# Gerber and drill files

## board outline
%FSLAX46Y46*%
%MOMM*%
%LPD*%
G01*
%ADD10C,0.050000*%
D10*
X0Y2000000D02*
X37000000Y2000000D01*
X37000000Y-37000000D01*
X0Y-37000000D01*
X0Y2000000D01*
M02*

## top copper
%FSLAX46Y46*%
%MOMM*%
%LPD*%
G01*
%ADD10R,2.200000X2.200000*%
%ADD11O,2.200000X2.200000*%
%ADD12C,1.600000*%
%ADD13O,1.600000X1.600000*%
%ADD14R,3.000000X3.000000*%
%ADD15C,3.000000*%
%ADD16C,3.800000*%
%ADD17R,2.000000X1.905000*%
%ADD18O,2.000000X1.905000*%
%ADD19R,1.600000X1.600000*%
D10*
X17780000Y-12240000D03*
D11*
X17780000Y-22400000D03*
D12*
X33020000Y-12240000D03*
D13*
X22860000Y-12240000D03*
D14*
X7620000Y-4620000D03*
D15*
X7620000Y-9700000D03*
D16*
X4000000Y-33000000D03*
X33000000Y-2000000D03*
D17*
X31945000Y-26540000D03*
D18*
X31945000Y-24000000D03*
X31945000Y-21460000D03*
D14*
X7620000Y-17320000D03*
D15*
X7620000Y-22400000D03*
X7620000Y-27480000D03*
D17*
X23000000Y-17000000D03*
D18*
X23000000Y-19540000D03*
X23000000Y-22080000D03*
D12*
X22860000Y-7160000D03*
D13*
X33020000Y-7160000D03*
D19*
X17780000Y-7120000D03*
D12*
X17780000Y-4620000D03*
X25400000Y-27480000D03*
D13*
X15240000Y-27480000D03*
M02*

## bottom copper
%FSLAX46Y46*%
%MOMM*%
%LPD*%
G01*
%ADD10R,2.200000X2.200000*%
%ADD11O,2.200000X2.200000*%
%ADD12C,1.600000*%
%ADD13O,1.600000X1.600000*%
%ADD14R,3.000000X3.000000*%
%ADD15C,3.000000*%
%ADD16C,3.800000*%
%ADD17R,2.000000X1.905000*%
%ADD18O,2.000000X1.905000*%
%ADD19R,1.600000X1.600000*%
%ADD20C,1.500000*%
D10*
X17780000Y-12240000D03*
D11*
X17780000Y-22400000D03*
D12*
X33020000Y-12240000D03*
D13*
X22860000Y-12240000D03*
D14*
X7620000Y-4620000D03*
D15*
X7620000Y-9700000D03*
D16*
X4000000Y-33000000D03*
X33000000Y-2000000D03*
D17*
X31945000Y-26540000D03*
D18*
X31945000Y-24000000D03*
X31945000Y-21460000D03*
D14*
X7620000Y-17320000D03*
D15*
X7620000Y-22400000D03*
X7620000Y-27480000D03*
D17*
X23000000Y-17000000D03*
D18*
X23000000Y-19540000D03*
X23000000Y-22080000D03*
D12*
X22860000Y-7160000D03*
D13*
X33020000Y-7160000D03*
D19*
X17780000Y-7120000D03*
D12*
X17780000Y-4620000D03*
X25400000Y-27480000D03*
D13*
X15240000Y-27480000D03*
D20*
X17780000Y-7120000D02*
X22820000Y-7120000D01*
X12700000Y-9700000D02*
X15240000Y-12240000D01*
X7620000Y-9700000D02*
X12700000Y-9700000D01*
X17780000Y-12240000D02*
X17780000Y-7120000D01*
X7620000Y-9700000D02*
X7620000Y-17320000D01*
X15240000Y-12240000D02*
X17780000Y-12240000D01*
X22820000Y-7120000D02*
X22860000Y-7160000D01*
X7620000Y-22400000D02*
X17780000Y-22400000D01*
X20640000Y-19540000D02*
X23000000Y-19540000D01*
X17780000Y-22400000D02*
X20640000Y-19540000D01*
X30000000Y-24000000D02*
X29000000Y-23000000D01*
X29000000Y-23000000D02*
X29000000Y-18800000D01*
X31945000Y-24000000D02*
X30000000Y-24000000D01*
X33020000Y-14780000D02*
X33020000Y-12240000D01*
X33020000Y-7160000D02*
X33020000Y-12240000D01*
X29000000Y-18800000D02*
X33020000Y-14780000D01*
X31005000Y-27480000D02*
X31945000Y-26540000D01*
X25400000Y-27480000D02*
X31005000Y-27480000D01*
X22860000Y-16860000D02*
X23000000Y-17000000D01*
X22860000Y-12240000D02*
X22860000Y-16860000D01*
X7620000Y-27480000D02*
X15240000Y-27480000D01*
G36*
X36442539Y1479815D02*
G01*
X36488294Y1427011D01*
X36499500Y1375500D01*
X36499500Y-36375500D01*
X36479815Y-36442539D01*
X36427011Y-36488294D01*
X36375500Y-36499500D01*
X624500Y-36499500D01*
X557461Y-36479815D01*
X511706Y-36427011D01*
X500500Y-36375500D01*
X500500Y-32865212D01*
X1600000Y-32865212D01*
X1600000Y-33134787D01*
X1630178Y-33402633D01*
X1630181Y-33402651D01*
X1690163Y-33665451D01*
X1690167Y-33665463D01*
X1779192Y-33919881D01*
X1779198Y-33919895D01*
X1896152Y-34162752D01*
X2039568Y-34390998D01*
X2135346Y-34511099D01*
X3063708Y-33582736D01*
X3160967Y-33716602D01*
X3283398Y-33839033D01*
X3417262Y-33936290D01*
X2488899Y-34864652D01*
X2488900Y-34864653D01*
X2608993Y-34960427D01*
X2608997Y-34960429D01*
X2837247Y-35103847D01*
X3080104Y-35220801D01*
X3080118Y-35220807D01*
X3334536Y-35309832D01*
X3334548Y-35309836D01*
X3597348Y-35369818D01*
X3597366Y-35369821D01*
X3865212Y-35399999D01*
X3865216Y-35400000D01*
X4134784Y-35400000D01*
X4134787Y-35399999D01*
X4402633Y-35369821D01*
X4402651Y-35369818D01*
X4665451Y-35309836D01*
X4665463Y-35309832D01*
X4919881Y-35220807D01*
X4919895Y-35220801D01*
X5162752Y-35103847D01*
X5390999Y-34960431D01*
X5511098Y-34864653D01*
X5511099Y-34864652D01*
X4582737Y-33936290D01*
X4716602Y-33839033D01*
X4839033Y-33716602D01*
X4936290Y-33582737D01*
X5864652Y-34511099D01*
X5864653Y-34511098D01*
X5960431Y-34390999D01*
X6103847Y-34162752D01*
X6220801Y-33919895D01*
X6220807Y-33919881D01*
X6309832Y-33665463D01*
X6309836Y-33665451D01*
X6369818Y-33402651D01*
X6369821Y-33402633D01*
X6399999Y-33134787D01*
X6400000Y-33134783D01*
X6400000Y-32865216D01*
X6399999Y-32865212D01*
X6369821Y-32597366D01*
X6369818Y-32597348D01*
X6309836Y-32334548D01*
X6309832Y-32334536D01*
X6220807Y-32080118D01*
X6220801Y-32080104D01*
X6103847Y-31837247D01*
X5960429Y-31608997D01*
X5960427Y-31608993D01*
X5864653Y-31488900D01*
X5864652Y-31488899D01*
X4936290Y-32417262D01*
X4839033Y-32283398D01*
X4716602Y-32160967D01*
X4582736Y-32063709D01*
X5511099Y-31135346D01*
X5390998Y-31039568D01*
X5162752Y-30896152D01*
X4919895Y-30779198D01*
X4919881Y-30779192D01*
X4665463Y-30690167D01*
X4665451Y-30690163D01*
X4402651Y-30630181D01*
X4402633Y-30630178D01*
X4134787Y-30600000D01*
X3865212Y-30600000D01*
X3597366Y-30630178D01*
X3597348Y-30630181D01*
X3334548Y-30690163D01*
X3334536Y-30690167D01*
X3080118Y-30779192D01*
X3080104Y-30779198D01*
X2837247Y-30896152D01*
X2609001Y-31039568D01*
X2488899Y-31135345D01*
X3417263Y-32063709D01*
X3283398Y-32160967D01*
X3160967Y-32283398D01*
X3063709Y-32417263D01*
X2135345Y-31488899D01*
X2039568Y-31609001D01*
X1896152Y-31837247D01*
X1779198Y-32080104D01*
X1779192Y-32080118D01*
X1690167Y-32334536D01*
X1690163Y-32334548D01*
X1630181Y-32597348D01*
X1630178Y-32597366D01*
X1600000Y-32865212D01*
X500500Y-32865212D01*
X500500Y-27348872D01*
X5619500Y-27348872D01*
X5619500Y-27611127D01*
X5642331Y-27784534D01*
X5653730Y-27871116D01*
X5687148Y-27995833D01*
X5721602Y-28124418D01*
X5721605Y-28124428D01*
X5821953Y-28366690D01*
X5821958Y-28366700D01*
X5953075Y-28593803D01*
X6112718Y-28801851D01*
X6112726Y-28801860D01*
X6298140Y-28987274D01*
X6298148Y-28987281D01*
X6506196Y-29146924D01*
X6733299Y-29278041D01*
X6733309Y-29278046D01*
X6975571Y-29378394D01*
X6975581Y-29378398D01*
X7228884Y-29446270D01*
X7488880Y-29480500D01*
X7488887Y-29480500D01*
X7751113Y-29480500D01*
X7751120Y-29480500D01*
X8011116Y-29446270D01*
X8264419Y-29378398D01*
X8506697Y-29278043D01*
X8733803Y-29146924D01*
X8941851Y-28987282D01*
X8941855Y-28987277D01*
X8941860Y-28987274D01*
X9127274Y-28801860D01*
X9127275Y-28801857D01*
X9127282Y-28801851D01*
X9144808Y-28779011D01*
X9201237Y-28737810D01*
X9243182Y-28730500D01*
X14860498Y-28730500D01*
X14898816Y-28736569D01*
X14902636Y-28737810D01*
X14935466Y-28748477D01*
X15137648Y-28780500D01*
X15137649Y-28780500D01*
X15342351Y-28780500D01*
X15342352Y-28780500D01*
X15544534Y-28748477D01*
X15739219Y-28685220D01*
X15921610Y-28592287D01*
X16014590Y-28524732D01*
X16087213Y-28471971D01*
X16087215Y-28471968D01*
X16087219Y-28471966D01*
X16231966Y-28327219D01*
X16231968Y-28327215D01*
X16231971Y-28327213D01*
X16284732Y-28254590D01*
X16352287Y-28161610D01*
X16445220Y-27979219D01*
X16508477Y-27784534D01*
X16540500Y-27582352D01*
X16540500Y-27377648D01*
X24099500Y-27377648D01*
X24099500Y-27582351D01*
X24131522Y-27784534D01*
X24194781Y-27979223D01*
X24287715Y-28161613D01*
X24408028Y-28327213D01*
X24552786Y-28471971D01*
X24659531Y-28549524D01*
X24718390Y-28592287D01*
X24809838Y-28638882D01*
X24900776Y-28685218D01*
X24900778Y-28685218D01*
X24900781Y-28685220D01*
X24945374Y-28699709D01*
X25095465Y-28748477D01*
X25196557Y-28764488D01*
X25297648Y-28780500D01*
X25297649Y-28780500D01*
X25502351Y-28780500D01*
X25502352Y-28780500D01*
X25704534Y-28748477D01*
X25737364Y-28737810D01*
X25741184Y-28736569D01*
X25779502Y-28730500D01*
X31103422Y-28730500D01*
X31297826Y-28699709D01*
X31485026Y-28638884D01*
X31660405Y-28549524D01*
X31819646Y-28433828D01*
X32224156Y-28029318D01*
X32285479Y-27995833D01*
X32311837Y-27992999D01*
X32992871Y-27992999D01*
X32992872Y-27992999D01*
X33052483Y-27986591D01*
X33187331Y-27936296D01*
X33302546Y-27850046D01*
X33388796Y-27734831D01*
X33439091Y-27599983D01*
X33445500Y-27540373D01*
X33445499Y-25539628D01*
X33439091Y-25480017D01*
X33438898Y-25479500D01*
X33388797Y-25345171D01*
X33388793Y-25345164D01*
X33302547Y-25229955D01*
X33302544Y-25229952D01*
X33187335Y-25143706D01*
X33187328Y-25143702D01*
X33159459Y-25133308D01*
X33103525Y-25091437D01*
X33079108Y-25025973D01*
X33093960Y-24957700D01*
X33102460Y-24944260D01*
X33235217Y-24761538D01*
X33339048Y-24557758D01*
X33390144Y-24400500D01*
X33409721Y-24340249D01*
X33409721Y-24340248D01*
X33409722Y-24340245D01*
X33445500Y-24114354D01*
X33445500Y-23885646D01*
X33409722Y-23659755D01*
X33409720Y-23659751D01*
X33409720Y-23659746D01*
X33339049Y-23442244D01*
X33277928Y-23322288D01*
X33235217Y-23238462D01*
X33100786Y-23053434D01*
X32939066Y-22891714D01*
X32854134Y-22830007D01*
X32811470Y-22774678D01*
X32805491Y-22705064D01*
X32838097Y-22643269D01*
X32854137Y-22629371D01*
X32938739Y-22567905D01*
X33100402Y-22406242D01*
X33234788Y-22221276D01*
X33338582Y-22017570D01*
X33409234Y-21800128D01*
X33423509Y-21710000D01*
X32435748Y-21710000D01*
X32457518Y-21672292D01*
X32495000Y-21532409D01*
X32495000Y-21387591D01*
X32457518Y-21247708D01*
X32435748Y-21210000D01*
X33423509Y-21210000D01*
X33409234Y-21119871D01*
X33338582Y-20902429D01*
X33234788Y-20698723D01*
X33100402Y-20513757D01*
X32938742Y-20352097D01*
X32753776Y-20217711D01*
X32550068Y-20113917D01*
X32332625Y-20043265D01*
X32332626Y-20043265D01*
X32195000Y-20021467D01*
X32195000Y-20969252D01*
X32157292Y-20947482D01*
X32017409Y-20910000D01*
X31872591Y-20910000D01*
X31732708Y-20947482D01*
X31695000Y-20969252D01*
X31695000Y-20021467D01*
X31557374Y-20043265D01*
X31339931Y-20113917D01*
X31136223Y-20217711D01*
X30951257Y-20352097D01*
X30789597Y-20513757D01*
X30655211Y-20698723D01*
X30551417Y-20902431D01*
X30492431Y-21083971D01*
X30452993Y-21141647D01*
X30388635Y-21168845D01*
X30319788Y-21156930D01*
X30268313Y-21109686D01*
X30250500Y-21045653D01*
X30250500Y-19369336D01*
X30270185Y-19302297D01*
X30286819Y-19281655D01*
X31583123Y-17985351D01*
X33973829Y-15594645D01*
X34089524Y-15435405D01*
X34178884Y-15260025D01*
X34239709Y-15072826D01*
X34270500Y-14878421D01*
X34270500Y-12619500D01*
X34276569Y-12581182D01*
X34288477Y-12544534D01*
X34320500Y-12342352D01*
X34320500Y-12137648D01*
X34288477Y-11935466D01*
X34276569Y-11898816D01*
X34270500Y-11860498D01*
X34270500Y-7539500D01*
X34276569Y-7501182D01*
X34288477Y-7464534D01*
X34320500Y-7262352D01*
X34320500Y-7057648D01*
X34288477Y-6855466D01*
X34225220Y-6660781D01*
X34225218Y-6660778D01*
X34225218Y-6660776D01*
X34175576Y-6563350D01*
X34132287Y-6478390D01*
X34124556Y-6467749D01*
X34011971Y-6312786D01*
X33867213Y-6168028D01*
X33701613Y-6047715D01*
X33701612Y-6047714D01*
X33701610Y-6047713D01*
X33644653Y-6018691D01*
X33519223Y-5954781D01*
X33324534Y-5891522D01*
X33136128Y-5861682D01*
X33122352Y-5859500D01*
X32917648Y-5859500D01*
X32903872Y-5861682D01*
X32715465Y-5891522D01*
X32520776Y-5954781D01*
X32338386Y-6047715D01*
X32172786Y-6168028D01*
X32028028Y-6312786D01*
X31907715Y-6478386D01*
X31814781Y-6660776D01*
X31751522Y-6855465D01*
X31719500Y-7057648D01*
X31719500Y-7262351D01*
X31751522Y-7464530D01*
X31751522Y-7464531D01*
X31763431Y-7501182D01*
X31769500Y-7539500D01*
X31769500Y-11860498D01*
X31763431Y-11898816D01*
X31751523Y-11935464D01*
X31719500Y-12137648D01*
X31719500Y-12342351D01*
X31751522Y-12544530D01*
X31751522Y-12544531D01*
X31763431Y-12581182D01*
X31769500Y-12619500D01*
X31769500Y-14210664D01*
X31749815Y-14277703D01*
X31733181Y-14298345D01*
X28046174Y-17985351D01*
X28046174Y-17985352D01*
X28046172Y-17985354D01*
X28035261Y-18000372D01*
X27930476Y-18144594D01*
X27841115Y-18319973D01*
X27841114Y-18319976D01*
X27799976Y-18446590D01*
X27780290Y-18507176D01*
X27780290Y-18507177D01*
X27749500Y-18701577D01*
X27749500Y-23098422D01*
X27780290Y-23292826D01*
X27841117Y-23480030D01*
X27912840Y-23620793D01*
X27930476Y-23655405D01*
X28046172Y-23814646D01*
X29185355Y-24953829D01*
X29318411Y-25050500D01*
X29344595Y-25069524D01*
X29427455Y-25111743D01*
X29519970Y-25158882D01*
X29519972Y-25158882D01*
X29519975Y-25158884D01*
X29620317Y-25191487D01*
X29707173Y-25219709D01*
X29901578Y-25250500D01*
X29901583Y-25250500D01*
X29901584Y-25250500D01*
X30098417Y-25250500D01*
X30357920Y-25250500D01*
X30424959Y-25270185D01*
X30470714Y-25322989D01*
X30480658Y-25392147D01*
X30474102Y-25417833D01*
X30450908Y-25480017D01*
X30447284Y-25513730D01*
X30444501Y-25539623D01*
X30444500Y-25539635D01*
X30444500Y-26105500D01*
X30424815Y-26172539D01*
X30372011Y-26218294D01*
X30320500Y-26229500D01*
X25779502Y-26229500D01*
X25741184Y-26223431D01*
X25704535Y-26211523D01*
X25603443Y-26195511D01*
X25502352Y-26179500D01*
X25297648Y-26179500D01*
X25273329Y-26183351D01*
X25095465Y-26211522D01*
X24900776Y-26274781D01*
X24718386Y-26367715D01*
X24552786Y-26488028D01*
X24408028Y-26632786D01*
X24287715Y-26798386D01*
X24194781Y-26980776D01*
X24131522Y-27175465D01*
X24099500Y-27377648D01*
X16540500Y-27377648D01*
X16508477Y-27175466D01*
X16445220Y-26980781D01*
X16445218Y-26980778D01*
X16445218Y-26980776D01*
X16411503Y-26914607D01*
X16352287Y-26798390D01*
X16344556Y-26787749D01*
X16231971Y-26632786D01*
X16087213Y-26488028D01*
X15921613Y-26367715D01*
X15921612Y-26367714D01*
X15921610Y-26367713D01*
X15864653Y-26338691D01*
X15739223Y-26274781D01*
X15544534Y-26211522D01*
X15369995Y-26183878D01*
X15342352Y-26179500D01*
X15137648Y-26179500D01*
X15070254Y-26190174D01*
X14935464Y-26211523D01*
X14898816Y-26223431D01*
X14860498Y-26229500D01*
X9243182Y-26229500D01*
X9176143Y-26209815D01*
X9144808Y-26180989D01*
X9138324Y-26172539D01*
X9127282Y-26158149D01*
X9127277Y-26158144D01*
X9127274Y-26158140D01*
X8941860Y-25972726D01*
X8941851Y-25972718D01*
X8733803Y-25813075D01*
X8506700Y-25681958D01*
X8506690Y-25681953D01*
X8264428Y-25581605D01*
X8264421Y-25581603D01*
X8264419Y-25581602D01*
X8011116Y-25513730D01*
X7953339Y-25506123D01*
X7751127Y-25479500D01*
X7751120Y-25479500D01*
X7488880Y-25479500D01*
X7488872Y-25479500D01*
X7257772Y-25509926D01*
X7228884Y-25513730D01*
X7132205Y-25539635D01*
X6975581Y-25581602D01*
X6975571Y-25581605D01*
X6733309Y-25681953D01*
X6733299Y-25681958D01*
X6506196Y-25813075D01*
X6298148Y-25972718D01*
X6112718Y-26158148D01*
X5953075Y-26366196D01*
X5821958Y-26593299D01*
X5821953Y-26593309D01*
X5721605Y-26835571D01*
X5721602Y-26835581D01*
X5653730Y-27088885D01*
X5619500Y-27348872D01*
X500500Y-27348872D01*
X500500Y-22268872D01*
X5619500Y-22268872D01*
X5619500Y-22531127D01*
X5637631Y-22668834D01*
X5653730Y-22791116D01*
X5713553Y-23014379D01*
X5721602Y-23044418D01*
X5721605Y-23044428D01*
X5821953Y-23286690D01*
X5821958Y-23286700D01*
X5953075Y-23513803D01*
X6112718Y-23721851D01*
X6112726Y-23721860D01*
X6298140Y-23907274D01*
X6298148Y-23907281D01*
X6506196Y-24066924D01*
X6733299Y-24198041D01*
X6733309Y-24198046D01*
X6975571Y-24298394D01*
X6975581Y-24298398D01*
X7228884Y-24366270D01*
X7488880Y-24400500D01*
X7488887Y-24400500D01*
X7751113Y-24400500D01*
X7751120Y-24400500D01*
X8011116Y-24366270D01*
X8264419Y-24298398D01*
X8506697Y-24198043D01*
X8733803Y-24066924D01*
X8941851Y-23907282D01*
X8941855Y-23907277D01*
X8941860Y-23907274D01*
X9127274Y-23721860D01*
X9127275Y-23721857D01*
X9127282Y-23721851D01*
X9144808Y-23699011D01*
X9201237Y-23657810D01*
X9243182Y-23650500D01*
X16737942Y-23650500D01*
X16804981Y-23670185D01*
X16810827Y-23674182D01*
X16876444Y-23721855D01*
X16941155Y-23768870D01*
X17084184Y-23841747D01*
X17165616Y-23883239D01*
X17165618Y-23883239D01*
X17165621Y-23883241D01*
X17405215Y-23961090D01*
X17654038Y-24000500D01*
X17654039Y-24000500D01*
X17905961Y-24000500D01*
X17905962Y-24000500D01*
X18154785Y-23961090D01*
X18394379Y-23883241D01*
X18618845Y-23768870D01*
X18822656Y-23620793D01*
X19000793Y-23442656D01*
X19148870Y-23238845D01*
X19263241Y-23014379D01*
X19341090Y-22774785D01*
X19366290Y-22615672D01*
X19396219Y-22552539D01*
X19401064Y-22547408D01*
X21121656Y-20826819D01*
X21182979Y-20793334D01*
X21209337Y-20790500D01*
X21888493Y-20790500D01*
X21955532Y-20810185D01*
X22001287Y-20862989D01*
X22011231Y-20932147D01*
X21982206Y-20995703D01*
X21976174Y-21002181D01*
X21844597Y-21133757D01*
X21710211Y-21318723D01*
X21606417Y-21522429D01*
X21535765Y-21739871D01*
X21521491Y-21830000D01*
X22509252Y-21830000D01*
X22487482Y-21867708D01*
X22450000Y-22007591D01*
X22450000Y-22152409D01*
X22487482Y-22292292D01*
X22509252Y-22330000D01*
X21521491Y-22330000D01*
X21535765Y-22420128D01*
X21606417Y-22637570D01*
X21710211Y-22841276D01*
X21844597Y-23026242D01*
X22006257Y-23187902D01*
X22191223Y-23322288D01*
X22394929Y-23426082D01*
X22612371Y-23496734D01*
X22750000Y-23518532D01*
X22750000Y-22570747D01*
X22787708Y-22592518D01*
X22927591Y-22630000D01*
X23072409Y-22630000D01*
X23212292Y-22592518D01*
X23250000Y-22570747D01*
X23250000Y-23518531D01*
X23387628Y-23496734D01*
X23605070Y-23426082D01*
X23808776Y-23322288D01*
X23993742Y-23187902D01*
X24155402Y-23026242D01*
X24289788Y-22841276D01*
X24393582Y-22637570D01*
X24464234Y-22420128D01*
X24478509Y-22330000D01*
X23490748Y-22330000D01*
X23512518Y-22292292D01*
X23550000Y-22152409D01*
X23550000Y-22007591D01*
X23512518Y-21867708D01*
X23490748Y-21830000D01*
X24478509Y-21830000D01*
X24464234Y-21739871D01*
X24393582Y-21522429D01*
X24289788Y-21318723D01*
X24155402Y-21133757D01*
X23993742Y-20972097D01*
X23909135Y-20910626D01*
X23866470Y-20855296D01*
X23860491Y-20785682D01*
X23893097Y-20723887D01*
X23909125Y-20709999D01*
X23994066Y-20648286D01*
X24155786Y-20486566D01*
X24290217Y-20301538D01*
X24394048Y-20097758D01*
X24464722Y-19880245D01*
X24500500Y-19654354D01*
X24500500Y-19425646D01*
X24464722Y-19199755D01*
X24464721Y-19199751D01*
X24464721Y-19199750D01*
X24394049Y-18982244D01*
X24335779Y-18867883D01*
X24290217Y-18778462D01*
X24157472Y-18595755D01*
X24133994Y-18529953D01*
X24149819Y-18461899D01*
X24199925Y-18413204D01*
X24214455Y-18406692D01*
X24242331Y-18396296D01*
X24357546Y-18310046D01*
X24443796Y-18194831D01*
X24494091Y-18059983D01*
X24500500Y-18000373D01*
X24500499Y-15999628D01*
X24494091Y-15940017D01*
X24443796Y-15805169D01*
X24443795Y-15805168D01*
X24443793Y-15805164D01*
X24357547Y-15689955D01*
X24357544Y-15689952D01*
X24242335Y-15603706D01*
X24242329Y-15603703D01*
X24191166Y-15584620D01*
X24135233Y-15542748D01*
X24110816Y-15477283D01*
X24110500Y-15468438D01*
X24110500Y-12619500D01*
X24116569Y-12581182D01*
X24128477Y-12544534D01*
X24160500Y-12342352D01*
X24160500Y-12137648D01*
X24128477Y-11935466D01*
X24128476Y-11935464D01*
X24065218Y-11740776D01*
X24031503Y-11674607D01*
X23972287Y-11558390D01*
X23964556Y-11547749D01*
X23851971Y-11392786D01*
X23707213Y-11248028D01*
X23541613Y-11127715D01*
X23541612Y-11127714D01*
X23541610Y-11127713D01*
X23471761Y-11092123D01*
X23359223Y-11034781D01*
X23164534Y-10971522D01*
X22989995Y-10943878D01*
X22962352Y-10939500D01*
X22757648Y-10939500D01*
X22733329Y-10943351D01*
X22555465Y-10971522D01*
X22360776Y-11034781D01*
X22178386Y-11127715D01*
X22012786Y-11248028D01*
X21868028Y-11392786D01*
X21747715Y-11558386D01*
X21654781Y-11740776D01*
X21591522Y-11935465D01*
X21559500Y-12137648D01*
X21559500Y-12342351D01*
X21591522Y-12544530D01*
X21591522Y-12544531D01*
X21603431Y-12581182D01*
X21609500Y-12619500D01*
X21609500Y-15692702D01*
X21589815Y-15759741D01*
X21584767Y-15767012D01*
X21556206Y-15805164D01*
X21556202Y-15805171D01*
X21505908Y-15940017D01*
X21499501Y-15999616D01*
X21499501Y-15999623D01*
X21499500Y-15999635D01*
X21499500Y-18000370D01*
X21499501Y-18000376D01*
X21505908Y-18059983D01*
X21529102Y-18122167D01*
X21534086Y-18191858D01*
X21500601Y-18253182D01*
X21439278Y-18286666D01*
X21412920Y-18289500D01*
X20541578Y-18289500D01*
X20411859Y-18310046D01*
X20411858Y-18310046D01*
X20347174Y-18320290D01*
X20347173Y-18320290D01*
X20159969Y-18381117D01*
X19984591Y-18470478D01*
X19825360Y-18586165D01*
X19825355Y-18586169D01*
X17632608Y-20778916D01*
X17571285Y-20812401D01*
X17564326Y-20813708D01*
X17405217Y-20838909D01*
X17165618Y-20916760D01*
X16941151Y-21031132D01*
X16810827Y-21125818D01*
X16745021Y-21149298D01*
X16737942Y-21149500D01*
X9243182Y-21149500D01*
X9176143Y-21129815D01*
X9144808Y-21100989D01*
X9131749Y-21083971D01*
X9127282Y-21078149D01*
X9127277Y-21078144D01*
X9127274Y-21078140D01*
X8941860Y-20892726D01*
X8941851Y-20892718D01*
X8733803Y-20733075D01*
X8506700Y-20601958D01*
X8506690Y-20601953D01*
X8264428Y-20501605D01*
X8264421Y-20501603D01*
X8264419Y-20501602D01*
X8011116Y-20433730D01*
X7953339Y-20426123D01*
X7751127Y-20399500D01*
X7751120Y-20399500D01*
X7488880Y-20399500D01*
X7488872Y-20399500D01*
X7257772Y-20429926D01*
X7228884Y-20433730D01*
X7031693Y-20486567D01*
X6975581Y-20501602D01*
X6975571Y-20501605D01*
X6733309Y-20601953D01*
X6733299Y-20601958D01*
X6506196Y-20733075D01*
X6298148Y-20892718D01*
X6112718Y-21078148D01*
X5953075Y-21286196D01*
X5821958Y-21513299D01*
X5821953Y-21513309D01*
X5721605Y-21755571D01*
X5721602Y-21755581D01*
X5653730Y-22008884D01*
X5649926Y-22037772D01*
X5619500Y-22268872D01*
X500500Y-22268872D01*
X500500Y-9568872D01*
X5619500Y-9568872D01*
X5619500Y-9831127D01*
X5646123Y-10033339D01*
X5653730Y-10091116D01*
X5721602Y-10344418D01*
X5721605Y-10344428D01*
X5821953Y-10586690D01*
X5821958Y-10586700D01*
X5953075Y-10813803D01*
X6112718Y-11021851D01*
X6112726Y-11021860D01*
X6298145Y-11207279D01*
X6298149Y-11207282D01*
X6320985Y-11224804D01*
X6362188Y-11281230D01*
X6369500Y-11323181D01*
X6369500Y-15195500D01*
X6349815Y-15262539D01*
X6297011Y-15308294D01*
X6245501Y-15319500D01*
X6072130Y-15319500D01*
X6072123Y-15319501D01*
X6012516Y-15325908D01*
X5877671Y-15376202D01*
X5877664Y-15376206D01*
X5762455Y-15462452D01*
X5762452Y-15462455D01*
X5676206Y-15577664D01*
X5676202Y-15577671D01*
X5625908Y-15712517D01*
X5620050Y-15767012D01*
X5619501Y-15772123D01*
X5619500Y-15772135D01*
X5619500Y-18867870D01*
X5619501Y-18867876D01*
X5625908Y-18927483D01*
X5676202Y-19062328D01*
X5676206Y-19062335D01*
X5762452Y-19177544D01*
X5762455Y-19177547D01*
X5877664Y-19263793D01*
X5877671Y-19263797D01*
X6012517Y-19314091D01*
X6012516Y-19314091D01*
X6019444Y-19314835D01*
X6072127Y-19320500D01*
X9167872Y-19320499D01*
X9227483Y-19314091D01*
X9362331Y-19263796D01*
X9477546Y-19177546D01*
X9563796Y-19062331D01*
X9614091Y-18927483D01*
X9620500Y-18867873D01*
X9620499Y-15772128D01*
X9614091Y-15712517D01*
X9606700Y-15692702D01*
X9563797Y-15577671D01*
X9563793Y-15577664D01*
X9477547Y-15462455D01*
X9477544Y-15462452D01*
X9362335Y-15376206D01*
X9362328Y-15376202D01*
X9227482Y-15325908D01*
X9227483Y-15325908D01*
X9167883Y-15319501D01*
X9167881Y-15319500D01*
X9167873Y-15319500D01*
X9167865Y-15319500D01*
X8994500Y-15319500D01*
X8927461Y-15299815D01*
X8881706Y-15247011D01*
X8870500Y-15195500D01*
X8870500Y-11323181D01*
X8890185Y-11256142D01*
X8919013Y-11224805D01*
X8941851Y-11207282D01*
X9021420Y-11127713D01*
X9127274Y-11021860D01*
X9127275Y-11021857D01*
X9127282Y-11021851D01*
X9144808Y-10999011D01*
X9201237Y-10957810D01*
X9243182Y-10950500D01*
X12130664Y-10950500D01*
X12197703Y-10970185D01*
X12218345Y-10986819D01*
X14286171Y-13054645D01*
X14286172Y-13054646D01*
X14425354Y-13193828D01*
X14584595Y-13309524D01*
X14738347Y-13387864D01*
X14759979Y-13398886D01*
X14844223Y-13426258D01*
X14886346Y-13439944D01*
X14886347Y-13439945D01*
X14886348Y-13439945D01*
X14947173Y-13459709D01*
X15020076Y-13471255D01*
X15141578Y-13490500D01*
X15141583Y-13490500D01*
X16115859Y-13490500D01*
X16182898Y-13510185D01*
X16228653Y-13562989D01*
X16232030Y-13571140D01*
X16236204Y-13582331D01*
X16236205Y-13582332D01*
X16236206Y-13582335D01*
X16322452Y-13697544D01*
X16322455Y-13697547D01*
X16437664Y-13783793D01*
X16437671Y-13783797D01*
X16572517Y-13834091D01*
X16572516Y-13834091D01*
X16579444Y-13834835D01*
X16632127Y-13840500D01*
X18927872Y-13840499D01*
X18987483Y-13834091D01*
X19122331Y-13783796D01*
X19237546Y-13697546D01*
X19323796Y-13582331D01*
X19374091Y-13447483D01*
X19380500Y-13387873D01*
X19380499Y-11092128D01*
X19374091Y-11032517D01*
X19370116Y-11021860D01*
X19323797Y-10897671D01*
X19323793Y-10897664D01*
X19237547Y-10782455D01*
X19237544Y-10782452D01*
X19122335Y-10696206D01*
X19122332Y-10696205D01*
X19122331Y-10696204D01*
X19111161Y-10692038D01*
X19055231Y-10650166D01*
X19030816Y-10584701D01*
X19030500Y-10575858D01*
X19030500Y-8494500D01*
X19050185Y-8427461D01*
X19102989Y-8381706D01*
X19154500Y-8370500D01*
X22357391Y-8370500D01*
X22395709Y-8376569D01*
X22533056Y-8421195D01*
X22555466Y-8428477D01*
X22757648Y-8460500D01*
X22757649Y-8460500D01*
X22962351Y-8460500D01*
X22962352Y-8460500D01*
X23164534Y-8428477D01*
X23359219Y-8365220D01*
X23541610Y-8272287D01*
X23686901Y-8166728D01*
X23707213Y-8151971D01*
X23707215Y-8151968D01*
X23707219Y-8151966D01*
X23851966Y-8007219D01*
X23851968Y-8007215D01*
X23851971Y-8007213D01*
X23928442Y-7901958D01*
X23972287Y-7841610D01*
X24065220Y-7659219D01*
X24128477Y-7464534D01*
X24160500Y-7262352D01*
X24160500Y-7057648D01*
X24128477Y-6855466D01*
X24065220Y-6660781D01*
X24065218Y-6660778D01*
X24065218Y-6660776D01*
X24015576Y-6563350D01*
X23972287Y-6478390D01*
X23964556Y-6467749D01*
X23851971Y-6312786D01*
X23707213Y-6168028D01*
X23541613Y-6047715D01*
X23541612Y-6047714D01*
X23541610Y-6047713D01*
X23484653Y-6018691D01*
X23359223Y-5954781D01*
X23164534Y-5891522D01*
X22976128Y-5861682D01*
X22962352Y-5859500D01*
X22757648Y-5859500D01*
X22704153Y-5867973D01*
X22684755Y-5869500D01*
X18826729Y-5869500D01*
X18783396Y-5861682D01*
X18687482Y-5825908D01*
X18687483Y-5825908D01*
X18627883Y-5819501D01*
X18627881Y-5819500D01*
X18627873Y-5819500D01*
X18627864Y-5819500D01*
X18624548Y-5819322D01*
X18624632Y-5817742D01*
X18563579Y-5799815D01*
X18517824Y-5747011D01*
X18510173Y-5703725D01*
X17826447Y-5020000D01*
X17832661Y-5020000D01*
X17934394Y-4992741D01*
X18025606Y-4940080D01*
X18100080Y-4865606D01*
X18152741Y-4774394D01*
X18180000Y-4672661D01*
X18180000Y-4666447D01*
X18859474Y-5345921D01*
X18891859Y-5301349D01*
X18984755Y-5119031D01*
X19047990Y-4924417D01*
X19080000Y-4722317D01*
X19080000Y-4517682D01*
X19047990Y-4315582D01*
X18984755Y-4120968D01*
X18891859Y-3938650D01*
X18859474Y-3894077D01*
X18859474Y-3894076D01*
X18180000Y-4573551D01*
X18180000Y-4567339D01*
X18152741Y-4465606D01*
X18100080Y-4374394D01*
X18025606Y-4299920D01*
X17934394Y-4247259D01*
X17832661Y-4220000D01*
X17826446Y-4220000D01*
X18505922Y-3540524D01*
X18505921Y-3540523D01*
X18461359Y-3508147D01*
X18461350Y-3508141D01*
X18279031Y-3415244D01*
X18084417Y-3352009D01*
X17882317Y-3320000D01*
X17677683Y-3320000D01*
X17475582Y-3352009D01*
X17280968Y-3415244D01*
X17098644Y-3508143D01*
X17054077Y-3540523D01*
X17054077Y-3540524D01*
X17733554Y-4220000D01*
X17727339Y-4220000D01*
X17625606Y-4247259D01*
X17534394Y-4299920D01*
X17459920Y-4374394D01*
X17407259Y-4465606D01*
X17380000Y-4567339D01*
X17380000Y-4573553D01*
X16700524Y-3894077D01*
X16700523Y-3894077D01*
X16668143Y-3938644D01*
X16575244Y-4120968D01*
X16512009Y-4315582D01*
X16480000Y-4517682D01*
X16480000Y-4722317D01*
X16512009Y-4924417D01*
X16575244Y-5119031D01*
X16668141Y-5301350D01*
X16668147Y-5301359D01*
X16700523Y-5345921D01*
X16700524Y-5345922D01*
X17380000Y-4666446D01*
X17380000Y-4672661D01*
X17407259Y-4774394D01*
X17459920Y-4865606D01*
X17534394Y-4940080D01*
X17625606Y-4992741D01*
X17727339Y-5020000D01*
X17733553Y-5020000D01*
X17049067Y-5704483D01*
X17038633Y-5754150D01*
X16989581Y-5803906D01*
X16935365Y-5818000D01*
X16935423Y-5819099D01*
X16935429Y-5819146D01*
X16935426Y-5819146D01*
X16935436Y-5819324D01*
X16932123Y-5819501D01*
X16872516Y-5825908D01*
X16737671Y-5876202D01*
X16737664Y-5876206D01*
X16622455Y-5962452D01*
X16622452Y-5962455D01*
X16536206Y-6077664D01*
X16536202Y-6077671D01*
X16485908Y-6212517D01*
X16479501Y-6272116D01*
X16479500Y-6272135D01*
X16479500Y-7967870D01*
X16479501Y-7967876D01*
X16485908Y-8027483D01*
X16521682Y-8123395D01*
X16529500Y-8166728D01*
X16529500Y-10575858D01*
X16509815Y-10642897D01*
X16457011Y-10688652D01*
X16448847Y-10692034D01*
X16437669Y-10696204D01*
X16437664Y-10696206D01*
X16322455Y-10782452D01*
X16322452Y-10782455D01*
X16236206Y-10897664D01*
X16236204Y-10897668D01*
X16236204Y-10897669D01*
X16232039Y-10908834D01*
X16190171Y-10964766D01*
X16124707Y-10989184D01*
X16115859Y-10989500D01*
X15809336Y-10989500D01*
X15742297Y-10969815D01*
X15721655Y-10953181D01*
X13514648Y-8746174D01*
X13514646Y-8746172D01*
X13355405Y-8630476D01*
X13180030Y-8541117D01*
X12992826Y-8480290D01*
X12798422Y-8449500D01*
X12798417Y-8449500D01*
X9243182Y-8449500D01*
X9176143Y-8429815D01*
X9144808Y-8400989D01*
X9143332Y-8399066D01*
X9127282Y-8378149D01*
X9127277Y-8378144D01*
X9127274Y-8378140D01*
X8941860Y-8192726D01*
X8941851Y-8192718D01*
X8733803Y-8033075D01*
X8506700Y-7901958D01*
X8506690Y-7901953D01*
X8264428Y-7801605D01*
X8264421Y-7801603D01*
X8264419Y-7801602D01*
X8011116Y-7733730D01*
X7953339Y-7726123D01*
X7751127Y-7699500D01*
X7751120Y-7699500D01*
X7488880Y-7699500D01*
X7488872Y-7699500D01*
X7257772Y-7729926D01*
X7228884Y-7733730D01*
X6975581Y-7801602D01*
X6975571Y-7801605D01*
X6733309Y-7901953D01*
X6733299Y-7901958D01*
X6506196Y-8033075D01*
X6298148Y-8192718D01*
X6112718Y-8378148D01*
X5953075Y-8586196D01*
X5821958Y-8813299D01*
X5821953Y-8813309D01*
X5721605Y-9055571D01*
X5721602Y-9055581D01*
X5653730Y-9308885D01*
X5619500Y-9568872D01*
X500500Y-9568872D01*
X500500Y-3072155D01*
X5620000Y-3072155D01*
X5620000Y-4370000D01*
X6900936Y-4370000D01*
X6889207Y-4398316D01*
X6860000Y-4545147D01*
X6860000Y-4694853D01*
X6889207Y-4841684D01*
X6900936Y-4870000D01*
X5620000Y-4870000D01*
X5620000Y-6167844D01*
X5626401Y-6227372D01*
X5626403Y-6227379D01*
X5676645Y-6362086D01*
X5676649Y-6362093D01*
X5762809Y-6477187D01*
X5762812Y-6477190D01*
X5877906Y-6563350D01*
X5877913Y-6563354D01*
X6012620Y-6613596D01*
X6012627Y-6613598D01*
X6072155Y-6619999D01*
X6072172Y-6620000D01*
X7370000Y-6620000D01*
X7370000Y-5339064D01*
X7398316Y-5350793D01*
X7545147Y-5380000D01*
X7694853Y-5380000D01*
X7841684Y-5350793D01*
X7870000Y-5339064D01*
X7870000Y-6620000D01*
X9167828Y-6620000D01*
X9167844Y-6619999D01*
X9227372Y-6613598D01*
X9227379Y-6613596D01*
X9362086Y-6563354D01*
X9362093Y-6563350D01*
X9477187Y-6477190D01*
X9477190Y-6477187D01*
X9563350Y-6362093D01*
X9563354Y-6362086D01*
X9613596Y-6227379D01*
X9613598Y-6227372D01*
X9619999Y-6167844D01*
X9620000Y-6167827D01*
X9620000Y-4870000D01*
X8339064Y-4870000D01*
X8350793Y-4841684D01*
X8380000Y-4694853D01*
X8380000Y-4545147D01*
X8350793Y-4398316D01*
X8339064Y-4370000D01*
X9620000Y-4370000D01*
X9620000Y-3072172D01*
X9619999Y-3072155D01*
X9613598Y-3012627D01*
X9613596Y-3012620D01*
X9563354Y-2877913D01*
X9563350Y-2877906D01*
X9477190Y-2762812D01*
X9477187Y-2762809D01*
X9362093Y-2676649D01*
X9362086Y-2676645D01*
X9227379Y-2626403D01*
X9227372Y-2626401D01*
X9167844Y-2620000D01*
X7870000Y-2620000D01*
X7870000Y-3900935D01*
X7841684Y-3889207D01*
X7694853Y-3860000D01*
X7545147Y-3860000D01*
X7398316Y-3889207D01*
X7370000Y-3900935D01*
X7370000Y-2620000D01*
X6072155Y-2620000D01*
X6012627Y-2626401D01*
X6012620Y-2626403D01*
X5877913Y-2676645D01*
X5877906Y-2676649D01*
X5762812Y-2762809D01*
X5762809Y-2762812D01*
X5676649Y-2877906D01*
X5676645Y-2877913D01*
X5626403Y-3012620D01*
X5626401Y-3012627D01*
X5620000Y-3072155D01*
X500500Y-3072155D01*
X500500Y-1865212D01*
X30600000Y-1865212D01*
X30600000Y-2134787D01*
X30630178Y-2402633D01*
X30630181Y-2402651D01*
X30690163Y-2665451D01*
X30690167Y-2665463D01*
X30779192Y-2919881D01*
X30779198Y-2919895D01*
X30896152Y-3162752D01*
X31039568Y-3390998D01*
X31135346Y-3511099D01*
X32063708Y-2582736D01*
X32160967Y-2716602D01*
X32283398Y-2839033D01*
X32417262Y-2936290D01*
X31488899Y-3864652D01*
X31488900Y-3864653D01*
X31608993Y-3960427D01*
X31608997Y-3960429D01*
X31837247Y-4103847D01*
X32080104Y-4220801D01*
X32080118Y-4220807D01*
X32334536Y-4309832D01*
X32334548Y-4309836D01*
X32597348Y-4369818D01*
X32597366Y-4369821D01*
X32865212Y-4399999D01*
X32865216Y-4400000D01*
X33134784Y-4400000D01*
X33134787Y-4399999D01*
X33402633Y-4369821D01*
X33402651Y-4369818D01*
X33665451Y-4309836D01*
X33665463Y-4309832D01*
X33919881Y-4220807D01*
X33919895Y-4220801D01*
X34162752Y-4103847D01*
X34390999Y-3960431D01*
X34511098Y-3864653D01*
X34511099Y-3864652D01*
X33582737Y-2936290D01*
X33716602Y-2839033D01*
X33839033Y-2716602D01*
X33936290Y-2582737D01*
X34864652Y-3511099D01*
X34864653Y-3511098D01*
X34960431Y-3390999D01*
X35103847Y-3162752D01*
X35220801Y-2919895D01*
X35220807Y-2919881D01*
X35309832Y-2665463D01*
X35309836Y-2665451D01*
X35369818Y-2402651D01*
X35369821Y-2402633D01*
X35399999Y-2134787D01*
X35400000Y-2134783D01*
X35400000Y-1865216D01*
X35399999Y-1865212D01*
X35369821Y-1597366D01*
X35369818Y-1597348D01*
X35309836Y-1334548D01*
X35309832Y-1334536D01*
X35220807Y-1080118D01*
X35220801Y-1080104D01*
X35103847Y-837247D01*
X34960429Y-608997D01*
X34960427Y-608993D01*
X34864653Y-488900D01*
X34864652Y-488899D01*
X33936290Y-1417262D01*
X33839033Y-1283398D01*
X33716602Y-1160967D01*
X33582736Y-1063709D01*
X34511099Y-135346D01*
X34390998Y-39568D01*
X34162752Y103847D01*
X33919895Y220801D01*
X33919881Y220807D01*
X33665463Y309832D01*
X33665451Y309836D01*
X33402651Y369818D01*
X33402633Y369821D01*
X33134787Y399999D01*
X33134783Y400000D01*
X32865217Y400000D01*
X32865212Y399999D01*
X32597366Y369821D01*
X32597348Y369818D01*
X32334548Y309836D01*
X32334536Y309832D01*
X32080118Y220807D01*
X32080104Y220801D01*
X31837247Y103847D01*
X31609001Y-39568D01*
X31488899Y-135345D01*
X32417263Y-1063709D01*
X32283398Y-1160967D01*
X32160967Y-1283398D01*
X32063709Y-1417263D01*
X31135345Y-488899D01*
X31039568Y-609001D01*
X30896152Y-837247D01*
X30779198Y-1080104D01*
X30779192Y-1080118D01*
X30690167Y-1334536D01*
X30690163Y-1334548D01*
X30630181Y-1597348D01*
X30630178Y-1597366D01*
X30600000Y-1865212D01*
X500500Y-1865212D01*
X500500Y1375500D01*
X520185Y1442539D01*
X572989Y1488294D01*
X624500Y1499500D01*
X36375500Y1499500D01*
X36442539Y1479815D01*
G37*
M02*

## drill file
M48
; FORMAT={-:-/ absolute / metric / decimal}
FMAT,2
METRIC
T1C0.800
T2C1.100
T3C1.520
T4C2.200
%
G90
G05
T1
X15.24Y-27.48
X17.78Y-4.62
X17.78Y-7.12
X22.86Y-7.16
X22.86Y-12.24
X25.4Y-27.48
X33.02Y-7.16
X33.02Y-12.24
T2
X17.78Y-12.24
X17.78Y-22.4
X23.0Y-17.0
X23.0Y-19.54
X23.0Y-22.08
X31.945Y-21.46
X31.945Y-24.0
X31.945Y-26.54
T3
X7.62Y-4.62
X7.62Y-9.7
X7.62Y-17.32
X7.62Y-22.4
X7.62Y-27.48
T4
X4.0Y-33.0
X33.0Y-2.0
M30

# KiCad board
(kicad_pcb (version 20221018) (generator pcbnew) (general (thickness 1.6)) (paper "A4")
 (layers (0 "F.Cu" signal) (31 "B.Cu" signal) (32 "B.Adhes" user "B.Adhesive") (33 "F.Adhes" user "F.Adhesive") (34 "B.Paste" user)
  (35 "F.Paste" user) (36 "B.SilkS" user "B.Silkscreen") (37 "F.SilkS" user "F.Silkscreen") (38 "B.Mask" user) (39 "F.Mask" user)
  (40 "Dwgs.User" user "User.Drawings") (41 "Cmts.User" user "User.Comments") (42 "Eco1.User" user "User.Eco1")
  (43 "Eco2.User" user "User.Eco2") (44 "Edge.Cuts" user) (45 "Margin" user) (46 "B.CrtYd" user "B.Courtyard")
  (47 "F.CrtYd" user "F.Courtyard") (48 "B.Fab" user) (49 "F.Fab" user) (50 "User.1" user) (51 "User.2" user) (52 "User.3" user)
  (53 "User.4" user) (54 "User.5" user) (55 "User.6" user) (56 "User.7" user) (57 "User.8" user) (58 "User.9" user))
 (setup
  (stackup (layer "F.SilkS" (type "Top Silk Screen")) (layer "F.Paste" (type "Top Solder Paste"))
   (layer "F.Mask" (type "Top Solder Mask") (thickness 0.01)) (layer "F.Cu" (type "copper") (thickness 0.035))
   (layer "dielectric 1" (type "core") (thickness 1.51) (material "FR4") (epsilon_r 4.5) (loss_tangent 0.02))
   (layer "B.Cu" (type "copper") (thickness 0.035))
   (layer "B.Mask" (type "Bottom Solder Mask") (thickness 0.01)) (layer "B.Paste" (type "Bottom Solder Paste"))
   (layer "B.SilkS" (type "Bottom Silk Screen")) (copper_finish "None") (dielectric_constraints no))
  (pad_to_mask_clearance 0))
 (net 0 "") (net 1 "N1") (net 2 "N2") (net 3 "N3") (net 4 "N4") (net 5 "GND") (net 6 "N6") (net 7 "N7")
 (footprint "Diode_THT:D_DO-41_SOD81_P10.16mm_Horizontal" (layer "F.Cu") (at 17.78 12.24 -90)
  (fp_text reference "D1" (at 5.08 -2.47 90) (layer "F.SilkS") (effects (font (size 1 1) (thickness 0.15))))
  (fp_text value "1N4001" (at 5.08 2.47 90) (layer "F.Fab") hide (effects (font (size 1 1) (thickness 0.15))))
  (pad "1" thru_hole rect (at 0 0 270) (size 2.2 2.2) (drill 1.1) (layers "*.Cu" "*.Mask") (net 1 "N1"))
  (pad "2" thru_hole oval (at 10.16 0 270) (size 2.2 2.2) (drill 1.1) (layers "*.Cu" "*.Mask") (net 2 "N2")))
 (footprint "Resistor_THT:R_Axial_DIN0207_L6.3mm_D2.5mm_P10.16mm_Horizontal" (layer "F.Cu") (at 33.02 12.24 180)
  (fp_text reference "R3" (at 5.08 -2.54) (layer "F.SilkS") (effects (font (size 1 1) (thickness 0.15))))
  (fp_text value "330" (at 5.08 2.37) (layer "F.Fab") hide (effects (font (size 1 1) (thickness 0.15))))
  (pad "1" thru_hole circle (at 0 0 180) (size 1.6 1.6) (drill 0.8) (layers "*.Cu" "*.Mask") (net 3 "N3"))
  (pad "2" thru_hole oval (at 10.16 0 180) (size 1.6 1.6) (drill 0.8) (layers "*.Cu" "*.Mask") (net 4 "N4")))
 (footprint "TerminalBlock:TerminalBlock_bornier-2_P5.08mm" (layer "F.Cu") (at 7.62 4.62 -90)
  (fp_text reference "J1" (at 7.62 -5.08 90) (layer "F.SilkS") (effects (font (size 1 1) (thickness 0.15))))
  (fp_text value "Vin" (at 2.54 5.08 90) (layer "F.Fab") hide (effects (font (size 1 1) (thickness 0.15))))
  (pad "1" thru_hole rect (at 0 0 270) (size 3 3) (drill 1.52) (layers "*.Cu" "*.Mask") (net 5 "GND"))
  (pad "2" thru_hole circle (at 5.08 0 270) (size 3 3) (drill 1.52) (layers "*.Cu" "*.Mask") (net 1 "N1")))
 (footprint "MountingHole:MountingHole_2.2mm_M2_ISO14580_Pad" (layer "F.Cu") (at 4 33)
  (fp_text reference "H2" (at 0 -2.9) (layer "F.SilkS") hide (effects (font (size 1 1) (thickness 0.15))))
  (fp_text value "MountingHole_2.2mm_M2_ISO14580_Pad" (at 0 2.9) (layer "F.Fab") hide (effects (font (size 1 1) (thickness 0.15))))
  (pad "2" thru_hole circle (at 0 0) (size 3.8 3.8) (drill 2.2) (layers "*.Cu" "*.Mask") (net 5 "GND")))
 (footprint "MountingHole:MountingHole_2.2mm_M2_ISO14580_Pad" (layer "F.Cu") (at 33 2)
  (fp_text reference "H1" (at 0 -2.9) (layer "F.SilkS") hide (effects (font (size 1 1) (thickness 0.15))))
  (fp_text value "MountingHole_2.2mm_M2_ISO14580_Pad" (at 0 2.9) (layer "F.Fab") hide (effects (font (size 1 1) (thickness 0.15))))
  (pad "1" thru_hole circle (at 0 0) (size 3.8 3.8) (drill 2.2) (layers "*.Cu" "*.Mask") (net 5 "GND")))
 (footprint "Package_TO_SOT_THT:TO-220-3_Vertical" (layer "F.Cu") (at 31.945 26.54 90)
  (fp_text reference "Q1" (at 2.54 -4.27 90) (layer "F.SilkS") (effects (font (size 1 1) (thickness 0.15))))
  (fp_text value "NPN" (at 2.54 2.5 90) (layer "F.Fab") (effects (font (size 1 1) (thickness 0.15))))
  (pad "1" thru_hole rect (at 0 0 90) (size 1.905 2) (drill 1.1) (layers "*.Cu" "*.Mask") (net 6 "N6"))
  (pad "2" thru_hole oval (at 2.54 0 90) (size 1.905 2) (drill 1.1) (layers "*.Cu" "*.Mask") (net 3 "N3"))
  (pad "3" thru_hole oval (at 5.08 0 90) (size 1.905 2) (drill 1.1) (layers "*.Cu" "*.Mask") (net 5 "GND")))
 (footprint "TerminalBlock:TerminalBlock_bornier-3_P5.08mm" (layer "F.Cu") (at 7.62 17.32 -90)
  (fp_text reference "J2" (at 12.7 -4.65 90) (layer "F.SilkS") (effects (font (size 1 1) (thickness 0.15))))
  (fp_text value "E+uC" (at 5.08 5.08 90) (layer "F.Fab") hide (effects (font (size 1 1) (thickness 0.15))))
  (pad "1" thru_hole rect (at 0 0 270) (size 3 3) (drill 1.52) (layers "*.Cu" "*.Mask") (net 1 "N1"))
  (pad "2" thru_hole circle (at 5.08 0 270) (size 3 3) (drill 1.52) (layers "*.Cu" "*.Mask") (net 2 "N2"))
  (pad "3" thru_hole circle (at 10.16 0 270) (size 3 3) (drill 1.52) (layers "*.Cu" "*.Mask") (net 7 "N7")))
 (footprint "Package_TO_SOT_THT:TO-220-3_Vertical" (layer "F.Cu") (at 23 17 -90)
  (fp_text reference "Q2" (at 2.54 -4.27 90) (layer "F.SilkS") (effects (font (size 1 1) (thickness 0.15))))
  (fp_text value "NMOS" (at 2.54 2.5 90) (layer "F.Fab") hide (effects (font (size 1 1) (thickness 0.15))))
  (pad "1" thru_hole rect (at 0 0 270) (size 1.905 2) (drill 1.1) (layers "*.Cu" "*.Mask") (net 4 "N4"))
  (pad "2" thru_hole oval (at 2.54 0 270) (size 1.905 2) (drill 1.1) (layers "*.Cu" "*.Mask") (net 2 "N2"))
  (pad "3" thru_hole oval (at 5.08 0 270) (size 1.905 2) (drill 1.1) (layers "*.Cu" "*.Mask") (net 5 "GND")))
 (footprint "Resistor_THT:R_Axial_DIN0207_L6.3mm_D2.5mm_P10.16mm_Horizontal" (layer "F.Cu") (at 22.86 7.16)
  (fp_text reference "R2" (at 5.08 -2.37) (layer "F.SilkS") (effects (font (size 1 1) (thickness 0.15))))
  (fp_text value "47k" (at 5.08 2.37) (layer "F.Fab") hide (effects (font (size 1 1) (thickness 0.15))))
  (pad "1" thru_hole circle (at 0 0) (size 1.6 1.6) (drill 0.8) (layers "*.Cu" "*.Mask") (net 1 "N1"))
  (pad "2" thru_hole oval (at 10.16 0) (size 1.6 1.6) (drill 0.8) (layers "*.Cu" "*.Mask") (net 3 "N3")))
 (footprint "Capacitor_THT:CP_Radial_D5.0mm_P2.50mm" (layer "F.Cu") (at 17.78 7.12 90)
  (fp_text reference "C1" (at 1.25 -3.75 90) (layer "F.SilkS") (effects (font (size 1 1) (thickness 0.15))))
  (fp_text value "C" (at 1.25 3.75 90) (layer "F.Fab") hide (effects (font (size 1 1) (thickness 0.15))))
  (pad "1" thru_hole rect (at 0 0 90) (size 1.6 1.6) (drill 0.8) (layers "*.Cu" "*.Mask") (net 1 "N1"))
  (pad "2" thru_hole circle (at 2.5 0 90) (size 1.6 1.6) (drill 0.8) (layers "*.Cu" "*.Mask") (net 5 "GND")))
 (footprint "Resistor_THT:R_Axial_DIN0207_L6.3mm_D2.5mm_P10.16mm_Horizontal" (layer "F.Cu") (at 25.4 27.48 180)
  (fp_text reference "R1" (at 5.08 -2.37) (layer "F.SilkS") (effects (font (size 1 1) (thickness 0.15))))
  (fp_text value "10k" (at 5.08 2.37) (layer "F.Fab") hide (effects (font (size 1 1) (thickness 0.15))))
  (pad "1" thru_hole circle (at 0 0 180) (size 1.6 1.6) (drill 0.8) (layers "*.Cu" "*.Mask") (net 6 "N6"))
  (pad "2" thru_hole oval (at 10.16 0 180) (size 1.6 1.6) (drill 0.8) (layers "*.Cu" "*.Mask") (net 7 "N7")))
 (gr_rect (start 0 -2) (end 37 37) (stroke (width 0.05) (type default)) (fill none) (layer "Edge.Cuts"))
 (segment (start 17.78 7.12) (end 22.82 7.12) (width 1.5) (layer "B.Cu") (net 1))
 (segment (start 12.7 9.7) (end 15.24 12.24) (width 1.5) (layer "B.Cu") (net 1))
 (segment (start 7.62 9.7) (end 12.7 9.7) (width 1.5) (layer "B.Cu") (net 1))
 (segment (start 17.78 12.24) (end 17.78 7.12) (width 1.5) (layer "B.Cu") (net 1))
 (segment (start 7.62 9.7) (end 7.62 17.32) (width 1.5) (layer "B.Cu") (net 1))
 (segment (start 15.24 12.24) (end 17.78 12.24) (width 1.5) (layer "B.Cu") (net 1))
 (segment (start 22.82 7.12) (end 22.86 7.16) (width 1.5) (layer "B.Cu") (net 1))
 (segment (start 7.62 22.4) (end 17.78 22.4) (width 1.5) (layer "B.Cu") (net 2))
 (segment (start 20.64 19.54) (end 23 19.54) (width 1.5) (layer "B.Cu") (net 2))
 (segment (start 17.78 22.4) (end 20.64 19.54) (width 1.5) (layer "B.Cu") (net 2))
 (segment (start 30 24) (end 29 23) (width 1.5) (layer "B.Cu") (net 3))
 (segment (start 29 23) (end 29 18.8) (width 1.5) (layer "B.Cu") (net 3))
 (segment (start 31.945 24) (end 30 24) (width 1.5) (layer "B.Cu") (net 3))
 (segment (start 33.02 14.78) (end 33.02 12.24) (width 1.5) (layer "B.Cu") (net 3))
 (segment (start 33.02 7.16) (end 33.02 12.24) (width 1.5) (layer "B.Cu") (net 3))
 (segment (start 29 18.8) (end 33.02 14.78) (width 1.5) (layer "B.Cu") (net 3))
 (segment (start 31.005 27.48) (end 31.945 26.54) (width 1.5) (layer "B.Cu") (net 6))
 (segment (start 25.4 27.48) (end 31.005 27.48) (width 1.5) (layer "B.Cu") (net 6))
 (segment (start 22.86 16.86) (end 23 17) (width 1.5) (layer "B.Cu") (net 4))
 (segment (start 22.86 12.24) (end 22.86 16.86) (width 1.5) (layer "B.Cu") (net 4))
 (segment (start 7.62 27.48) (end 15.24 27.48) (width 1.5) (layer "B.Cu") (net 7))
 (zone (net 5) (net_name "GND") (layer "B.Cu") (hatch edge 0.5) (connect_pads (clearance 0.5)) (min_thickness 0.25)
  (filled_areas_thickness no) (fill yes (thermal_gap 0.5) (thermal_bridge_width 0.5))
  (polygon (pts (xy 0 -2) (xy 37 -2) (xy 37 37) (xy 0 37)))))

